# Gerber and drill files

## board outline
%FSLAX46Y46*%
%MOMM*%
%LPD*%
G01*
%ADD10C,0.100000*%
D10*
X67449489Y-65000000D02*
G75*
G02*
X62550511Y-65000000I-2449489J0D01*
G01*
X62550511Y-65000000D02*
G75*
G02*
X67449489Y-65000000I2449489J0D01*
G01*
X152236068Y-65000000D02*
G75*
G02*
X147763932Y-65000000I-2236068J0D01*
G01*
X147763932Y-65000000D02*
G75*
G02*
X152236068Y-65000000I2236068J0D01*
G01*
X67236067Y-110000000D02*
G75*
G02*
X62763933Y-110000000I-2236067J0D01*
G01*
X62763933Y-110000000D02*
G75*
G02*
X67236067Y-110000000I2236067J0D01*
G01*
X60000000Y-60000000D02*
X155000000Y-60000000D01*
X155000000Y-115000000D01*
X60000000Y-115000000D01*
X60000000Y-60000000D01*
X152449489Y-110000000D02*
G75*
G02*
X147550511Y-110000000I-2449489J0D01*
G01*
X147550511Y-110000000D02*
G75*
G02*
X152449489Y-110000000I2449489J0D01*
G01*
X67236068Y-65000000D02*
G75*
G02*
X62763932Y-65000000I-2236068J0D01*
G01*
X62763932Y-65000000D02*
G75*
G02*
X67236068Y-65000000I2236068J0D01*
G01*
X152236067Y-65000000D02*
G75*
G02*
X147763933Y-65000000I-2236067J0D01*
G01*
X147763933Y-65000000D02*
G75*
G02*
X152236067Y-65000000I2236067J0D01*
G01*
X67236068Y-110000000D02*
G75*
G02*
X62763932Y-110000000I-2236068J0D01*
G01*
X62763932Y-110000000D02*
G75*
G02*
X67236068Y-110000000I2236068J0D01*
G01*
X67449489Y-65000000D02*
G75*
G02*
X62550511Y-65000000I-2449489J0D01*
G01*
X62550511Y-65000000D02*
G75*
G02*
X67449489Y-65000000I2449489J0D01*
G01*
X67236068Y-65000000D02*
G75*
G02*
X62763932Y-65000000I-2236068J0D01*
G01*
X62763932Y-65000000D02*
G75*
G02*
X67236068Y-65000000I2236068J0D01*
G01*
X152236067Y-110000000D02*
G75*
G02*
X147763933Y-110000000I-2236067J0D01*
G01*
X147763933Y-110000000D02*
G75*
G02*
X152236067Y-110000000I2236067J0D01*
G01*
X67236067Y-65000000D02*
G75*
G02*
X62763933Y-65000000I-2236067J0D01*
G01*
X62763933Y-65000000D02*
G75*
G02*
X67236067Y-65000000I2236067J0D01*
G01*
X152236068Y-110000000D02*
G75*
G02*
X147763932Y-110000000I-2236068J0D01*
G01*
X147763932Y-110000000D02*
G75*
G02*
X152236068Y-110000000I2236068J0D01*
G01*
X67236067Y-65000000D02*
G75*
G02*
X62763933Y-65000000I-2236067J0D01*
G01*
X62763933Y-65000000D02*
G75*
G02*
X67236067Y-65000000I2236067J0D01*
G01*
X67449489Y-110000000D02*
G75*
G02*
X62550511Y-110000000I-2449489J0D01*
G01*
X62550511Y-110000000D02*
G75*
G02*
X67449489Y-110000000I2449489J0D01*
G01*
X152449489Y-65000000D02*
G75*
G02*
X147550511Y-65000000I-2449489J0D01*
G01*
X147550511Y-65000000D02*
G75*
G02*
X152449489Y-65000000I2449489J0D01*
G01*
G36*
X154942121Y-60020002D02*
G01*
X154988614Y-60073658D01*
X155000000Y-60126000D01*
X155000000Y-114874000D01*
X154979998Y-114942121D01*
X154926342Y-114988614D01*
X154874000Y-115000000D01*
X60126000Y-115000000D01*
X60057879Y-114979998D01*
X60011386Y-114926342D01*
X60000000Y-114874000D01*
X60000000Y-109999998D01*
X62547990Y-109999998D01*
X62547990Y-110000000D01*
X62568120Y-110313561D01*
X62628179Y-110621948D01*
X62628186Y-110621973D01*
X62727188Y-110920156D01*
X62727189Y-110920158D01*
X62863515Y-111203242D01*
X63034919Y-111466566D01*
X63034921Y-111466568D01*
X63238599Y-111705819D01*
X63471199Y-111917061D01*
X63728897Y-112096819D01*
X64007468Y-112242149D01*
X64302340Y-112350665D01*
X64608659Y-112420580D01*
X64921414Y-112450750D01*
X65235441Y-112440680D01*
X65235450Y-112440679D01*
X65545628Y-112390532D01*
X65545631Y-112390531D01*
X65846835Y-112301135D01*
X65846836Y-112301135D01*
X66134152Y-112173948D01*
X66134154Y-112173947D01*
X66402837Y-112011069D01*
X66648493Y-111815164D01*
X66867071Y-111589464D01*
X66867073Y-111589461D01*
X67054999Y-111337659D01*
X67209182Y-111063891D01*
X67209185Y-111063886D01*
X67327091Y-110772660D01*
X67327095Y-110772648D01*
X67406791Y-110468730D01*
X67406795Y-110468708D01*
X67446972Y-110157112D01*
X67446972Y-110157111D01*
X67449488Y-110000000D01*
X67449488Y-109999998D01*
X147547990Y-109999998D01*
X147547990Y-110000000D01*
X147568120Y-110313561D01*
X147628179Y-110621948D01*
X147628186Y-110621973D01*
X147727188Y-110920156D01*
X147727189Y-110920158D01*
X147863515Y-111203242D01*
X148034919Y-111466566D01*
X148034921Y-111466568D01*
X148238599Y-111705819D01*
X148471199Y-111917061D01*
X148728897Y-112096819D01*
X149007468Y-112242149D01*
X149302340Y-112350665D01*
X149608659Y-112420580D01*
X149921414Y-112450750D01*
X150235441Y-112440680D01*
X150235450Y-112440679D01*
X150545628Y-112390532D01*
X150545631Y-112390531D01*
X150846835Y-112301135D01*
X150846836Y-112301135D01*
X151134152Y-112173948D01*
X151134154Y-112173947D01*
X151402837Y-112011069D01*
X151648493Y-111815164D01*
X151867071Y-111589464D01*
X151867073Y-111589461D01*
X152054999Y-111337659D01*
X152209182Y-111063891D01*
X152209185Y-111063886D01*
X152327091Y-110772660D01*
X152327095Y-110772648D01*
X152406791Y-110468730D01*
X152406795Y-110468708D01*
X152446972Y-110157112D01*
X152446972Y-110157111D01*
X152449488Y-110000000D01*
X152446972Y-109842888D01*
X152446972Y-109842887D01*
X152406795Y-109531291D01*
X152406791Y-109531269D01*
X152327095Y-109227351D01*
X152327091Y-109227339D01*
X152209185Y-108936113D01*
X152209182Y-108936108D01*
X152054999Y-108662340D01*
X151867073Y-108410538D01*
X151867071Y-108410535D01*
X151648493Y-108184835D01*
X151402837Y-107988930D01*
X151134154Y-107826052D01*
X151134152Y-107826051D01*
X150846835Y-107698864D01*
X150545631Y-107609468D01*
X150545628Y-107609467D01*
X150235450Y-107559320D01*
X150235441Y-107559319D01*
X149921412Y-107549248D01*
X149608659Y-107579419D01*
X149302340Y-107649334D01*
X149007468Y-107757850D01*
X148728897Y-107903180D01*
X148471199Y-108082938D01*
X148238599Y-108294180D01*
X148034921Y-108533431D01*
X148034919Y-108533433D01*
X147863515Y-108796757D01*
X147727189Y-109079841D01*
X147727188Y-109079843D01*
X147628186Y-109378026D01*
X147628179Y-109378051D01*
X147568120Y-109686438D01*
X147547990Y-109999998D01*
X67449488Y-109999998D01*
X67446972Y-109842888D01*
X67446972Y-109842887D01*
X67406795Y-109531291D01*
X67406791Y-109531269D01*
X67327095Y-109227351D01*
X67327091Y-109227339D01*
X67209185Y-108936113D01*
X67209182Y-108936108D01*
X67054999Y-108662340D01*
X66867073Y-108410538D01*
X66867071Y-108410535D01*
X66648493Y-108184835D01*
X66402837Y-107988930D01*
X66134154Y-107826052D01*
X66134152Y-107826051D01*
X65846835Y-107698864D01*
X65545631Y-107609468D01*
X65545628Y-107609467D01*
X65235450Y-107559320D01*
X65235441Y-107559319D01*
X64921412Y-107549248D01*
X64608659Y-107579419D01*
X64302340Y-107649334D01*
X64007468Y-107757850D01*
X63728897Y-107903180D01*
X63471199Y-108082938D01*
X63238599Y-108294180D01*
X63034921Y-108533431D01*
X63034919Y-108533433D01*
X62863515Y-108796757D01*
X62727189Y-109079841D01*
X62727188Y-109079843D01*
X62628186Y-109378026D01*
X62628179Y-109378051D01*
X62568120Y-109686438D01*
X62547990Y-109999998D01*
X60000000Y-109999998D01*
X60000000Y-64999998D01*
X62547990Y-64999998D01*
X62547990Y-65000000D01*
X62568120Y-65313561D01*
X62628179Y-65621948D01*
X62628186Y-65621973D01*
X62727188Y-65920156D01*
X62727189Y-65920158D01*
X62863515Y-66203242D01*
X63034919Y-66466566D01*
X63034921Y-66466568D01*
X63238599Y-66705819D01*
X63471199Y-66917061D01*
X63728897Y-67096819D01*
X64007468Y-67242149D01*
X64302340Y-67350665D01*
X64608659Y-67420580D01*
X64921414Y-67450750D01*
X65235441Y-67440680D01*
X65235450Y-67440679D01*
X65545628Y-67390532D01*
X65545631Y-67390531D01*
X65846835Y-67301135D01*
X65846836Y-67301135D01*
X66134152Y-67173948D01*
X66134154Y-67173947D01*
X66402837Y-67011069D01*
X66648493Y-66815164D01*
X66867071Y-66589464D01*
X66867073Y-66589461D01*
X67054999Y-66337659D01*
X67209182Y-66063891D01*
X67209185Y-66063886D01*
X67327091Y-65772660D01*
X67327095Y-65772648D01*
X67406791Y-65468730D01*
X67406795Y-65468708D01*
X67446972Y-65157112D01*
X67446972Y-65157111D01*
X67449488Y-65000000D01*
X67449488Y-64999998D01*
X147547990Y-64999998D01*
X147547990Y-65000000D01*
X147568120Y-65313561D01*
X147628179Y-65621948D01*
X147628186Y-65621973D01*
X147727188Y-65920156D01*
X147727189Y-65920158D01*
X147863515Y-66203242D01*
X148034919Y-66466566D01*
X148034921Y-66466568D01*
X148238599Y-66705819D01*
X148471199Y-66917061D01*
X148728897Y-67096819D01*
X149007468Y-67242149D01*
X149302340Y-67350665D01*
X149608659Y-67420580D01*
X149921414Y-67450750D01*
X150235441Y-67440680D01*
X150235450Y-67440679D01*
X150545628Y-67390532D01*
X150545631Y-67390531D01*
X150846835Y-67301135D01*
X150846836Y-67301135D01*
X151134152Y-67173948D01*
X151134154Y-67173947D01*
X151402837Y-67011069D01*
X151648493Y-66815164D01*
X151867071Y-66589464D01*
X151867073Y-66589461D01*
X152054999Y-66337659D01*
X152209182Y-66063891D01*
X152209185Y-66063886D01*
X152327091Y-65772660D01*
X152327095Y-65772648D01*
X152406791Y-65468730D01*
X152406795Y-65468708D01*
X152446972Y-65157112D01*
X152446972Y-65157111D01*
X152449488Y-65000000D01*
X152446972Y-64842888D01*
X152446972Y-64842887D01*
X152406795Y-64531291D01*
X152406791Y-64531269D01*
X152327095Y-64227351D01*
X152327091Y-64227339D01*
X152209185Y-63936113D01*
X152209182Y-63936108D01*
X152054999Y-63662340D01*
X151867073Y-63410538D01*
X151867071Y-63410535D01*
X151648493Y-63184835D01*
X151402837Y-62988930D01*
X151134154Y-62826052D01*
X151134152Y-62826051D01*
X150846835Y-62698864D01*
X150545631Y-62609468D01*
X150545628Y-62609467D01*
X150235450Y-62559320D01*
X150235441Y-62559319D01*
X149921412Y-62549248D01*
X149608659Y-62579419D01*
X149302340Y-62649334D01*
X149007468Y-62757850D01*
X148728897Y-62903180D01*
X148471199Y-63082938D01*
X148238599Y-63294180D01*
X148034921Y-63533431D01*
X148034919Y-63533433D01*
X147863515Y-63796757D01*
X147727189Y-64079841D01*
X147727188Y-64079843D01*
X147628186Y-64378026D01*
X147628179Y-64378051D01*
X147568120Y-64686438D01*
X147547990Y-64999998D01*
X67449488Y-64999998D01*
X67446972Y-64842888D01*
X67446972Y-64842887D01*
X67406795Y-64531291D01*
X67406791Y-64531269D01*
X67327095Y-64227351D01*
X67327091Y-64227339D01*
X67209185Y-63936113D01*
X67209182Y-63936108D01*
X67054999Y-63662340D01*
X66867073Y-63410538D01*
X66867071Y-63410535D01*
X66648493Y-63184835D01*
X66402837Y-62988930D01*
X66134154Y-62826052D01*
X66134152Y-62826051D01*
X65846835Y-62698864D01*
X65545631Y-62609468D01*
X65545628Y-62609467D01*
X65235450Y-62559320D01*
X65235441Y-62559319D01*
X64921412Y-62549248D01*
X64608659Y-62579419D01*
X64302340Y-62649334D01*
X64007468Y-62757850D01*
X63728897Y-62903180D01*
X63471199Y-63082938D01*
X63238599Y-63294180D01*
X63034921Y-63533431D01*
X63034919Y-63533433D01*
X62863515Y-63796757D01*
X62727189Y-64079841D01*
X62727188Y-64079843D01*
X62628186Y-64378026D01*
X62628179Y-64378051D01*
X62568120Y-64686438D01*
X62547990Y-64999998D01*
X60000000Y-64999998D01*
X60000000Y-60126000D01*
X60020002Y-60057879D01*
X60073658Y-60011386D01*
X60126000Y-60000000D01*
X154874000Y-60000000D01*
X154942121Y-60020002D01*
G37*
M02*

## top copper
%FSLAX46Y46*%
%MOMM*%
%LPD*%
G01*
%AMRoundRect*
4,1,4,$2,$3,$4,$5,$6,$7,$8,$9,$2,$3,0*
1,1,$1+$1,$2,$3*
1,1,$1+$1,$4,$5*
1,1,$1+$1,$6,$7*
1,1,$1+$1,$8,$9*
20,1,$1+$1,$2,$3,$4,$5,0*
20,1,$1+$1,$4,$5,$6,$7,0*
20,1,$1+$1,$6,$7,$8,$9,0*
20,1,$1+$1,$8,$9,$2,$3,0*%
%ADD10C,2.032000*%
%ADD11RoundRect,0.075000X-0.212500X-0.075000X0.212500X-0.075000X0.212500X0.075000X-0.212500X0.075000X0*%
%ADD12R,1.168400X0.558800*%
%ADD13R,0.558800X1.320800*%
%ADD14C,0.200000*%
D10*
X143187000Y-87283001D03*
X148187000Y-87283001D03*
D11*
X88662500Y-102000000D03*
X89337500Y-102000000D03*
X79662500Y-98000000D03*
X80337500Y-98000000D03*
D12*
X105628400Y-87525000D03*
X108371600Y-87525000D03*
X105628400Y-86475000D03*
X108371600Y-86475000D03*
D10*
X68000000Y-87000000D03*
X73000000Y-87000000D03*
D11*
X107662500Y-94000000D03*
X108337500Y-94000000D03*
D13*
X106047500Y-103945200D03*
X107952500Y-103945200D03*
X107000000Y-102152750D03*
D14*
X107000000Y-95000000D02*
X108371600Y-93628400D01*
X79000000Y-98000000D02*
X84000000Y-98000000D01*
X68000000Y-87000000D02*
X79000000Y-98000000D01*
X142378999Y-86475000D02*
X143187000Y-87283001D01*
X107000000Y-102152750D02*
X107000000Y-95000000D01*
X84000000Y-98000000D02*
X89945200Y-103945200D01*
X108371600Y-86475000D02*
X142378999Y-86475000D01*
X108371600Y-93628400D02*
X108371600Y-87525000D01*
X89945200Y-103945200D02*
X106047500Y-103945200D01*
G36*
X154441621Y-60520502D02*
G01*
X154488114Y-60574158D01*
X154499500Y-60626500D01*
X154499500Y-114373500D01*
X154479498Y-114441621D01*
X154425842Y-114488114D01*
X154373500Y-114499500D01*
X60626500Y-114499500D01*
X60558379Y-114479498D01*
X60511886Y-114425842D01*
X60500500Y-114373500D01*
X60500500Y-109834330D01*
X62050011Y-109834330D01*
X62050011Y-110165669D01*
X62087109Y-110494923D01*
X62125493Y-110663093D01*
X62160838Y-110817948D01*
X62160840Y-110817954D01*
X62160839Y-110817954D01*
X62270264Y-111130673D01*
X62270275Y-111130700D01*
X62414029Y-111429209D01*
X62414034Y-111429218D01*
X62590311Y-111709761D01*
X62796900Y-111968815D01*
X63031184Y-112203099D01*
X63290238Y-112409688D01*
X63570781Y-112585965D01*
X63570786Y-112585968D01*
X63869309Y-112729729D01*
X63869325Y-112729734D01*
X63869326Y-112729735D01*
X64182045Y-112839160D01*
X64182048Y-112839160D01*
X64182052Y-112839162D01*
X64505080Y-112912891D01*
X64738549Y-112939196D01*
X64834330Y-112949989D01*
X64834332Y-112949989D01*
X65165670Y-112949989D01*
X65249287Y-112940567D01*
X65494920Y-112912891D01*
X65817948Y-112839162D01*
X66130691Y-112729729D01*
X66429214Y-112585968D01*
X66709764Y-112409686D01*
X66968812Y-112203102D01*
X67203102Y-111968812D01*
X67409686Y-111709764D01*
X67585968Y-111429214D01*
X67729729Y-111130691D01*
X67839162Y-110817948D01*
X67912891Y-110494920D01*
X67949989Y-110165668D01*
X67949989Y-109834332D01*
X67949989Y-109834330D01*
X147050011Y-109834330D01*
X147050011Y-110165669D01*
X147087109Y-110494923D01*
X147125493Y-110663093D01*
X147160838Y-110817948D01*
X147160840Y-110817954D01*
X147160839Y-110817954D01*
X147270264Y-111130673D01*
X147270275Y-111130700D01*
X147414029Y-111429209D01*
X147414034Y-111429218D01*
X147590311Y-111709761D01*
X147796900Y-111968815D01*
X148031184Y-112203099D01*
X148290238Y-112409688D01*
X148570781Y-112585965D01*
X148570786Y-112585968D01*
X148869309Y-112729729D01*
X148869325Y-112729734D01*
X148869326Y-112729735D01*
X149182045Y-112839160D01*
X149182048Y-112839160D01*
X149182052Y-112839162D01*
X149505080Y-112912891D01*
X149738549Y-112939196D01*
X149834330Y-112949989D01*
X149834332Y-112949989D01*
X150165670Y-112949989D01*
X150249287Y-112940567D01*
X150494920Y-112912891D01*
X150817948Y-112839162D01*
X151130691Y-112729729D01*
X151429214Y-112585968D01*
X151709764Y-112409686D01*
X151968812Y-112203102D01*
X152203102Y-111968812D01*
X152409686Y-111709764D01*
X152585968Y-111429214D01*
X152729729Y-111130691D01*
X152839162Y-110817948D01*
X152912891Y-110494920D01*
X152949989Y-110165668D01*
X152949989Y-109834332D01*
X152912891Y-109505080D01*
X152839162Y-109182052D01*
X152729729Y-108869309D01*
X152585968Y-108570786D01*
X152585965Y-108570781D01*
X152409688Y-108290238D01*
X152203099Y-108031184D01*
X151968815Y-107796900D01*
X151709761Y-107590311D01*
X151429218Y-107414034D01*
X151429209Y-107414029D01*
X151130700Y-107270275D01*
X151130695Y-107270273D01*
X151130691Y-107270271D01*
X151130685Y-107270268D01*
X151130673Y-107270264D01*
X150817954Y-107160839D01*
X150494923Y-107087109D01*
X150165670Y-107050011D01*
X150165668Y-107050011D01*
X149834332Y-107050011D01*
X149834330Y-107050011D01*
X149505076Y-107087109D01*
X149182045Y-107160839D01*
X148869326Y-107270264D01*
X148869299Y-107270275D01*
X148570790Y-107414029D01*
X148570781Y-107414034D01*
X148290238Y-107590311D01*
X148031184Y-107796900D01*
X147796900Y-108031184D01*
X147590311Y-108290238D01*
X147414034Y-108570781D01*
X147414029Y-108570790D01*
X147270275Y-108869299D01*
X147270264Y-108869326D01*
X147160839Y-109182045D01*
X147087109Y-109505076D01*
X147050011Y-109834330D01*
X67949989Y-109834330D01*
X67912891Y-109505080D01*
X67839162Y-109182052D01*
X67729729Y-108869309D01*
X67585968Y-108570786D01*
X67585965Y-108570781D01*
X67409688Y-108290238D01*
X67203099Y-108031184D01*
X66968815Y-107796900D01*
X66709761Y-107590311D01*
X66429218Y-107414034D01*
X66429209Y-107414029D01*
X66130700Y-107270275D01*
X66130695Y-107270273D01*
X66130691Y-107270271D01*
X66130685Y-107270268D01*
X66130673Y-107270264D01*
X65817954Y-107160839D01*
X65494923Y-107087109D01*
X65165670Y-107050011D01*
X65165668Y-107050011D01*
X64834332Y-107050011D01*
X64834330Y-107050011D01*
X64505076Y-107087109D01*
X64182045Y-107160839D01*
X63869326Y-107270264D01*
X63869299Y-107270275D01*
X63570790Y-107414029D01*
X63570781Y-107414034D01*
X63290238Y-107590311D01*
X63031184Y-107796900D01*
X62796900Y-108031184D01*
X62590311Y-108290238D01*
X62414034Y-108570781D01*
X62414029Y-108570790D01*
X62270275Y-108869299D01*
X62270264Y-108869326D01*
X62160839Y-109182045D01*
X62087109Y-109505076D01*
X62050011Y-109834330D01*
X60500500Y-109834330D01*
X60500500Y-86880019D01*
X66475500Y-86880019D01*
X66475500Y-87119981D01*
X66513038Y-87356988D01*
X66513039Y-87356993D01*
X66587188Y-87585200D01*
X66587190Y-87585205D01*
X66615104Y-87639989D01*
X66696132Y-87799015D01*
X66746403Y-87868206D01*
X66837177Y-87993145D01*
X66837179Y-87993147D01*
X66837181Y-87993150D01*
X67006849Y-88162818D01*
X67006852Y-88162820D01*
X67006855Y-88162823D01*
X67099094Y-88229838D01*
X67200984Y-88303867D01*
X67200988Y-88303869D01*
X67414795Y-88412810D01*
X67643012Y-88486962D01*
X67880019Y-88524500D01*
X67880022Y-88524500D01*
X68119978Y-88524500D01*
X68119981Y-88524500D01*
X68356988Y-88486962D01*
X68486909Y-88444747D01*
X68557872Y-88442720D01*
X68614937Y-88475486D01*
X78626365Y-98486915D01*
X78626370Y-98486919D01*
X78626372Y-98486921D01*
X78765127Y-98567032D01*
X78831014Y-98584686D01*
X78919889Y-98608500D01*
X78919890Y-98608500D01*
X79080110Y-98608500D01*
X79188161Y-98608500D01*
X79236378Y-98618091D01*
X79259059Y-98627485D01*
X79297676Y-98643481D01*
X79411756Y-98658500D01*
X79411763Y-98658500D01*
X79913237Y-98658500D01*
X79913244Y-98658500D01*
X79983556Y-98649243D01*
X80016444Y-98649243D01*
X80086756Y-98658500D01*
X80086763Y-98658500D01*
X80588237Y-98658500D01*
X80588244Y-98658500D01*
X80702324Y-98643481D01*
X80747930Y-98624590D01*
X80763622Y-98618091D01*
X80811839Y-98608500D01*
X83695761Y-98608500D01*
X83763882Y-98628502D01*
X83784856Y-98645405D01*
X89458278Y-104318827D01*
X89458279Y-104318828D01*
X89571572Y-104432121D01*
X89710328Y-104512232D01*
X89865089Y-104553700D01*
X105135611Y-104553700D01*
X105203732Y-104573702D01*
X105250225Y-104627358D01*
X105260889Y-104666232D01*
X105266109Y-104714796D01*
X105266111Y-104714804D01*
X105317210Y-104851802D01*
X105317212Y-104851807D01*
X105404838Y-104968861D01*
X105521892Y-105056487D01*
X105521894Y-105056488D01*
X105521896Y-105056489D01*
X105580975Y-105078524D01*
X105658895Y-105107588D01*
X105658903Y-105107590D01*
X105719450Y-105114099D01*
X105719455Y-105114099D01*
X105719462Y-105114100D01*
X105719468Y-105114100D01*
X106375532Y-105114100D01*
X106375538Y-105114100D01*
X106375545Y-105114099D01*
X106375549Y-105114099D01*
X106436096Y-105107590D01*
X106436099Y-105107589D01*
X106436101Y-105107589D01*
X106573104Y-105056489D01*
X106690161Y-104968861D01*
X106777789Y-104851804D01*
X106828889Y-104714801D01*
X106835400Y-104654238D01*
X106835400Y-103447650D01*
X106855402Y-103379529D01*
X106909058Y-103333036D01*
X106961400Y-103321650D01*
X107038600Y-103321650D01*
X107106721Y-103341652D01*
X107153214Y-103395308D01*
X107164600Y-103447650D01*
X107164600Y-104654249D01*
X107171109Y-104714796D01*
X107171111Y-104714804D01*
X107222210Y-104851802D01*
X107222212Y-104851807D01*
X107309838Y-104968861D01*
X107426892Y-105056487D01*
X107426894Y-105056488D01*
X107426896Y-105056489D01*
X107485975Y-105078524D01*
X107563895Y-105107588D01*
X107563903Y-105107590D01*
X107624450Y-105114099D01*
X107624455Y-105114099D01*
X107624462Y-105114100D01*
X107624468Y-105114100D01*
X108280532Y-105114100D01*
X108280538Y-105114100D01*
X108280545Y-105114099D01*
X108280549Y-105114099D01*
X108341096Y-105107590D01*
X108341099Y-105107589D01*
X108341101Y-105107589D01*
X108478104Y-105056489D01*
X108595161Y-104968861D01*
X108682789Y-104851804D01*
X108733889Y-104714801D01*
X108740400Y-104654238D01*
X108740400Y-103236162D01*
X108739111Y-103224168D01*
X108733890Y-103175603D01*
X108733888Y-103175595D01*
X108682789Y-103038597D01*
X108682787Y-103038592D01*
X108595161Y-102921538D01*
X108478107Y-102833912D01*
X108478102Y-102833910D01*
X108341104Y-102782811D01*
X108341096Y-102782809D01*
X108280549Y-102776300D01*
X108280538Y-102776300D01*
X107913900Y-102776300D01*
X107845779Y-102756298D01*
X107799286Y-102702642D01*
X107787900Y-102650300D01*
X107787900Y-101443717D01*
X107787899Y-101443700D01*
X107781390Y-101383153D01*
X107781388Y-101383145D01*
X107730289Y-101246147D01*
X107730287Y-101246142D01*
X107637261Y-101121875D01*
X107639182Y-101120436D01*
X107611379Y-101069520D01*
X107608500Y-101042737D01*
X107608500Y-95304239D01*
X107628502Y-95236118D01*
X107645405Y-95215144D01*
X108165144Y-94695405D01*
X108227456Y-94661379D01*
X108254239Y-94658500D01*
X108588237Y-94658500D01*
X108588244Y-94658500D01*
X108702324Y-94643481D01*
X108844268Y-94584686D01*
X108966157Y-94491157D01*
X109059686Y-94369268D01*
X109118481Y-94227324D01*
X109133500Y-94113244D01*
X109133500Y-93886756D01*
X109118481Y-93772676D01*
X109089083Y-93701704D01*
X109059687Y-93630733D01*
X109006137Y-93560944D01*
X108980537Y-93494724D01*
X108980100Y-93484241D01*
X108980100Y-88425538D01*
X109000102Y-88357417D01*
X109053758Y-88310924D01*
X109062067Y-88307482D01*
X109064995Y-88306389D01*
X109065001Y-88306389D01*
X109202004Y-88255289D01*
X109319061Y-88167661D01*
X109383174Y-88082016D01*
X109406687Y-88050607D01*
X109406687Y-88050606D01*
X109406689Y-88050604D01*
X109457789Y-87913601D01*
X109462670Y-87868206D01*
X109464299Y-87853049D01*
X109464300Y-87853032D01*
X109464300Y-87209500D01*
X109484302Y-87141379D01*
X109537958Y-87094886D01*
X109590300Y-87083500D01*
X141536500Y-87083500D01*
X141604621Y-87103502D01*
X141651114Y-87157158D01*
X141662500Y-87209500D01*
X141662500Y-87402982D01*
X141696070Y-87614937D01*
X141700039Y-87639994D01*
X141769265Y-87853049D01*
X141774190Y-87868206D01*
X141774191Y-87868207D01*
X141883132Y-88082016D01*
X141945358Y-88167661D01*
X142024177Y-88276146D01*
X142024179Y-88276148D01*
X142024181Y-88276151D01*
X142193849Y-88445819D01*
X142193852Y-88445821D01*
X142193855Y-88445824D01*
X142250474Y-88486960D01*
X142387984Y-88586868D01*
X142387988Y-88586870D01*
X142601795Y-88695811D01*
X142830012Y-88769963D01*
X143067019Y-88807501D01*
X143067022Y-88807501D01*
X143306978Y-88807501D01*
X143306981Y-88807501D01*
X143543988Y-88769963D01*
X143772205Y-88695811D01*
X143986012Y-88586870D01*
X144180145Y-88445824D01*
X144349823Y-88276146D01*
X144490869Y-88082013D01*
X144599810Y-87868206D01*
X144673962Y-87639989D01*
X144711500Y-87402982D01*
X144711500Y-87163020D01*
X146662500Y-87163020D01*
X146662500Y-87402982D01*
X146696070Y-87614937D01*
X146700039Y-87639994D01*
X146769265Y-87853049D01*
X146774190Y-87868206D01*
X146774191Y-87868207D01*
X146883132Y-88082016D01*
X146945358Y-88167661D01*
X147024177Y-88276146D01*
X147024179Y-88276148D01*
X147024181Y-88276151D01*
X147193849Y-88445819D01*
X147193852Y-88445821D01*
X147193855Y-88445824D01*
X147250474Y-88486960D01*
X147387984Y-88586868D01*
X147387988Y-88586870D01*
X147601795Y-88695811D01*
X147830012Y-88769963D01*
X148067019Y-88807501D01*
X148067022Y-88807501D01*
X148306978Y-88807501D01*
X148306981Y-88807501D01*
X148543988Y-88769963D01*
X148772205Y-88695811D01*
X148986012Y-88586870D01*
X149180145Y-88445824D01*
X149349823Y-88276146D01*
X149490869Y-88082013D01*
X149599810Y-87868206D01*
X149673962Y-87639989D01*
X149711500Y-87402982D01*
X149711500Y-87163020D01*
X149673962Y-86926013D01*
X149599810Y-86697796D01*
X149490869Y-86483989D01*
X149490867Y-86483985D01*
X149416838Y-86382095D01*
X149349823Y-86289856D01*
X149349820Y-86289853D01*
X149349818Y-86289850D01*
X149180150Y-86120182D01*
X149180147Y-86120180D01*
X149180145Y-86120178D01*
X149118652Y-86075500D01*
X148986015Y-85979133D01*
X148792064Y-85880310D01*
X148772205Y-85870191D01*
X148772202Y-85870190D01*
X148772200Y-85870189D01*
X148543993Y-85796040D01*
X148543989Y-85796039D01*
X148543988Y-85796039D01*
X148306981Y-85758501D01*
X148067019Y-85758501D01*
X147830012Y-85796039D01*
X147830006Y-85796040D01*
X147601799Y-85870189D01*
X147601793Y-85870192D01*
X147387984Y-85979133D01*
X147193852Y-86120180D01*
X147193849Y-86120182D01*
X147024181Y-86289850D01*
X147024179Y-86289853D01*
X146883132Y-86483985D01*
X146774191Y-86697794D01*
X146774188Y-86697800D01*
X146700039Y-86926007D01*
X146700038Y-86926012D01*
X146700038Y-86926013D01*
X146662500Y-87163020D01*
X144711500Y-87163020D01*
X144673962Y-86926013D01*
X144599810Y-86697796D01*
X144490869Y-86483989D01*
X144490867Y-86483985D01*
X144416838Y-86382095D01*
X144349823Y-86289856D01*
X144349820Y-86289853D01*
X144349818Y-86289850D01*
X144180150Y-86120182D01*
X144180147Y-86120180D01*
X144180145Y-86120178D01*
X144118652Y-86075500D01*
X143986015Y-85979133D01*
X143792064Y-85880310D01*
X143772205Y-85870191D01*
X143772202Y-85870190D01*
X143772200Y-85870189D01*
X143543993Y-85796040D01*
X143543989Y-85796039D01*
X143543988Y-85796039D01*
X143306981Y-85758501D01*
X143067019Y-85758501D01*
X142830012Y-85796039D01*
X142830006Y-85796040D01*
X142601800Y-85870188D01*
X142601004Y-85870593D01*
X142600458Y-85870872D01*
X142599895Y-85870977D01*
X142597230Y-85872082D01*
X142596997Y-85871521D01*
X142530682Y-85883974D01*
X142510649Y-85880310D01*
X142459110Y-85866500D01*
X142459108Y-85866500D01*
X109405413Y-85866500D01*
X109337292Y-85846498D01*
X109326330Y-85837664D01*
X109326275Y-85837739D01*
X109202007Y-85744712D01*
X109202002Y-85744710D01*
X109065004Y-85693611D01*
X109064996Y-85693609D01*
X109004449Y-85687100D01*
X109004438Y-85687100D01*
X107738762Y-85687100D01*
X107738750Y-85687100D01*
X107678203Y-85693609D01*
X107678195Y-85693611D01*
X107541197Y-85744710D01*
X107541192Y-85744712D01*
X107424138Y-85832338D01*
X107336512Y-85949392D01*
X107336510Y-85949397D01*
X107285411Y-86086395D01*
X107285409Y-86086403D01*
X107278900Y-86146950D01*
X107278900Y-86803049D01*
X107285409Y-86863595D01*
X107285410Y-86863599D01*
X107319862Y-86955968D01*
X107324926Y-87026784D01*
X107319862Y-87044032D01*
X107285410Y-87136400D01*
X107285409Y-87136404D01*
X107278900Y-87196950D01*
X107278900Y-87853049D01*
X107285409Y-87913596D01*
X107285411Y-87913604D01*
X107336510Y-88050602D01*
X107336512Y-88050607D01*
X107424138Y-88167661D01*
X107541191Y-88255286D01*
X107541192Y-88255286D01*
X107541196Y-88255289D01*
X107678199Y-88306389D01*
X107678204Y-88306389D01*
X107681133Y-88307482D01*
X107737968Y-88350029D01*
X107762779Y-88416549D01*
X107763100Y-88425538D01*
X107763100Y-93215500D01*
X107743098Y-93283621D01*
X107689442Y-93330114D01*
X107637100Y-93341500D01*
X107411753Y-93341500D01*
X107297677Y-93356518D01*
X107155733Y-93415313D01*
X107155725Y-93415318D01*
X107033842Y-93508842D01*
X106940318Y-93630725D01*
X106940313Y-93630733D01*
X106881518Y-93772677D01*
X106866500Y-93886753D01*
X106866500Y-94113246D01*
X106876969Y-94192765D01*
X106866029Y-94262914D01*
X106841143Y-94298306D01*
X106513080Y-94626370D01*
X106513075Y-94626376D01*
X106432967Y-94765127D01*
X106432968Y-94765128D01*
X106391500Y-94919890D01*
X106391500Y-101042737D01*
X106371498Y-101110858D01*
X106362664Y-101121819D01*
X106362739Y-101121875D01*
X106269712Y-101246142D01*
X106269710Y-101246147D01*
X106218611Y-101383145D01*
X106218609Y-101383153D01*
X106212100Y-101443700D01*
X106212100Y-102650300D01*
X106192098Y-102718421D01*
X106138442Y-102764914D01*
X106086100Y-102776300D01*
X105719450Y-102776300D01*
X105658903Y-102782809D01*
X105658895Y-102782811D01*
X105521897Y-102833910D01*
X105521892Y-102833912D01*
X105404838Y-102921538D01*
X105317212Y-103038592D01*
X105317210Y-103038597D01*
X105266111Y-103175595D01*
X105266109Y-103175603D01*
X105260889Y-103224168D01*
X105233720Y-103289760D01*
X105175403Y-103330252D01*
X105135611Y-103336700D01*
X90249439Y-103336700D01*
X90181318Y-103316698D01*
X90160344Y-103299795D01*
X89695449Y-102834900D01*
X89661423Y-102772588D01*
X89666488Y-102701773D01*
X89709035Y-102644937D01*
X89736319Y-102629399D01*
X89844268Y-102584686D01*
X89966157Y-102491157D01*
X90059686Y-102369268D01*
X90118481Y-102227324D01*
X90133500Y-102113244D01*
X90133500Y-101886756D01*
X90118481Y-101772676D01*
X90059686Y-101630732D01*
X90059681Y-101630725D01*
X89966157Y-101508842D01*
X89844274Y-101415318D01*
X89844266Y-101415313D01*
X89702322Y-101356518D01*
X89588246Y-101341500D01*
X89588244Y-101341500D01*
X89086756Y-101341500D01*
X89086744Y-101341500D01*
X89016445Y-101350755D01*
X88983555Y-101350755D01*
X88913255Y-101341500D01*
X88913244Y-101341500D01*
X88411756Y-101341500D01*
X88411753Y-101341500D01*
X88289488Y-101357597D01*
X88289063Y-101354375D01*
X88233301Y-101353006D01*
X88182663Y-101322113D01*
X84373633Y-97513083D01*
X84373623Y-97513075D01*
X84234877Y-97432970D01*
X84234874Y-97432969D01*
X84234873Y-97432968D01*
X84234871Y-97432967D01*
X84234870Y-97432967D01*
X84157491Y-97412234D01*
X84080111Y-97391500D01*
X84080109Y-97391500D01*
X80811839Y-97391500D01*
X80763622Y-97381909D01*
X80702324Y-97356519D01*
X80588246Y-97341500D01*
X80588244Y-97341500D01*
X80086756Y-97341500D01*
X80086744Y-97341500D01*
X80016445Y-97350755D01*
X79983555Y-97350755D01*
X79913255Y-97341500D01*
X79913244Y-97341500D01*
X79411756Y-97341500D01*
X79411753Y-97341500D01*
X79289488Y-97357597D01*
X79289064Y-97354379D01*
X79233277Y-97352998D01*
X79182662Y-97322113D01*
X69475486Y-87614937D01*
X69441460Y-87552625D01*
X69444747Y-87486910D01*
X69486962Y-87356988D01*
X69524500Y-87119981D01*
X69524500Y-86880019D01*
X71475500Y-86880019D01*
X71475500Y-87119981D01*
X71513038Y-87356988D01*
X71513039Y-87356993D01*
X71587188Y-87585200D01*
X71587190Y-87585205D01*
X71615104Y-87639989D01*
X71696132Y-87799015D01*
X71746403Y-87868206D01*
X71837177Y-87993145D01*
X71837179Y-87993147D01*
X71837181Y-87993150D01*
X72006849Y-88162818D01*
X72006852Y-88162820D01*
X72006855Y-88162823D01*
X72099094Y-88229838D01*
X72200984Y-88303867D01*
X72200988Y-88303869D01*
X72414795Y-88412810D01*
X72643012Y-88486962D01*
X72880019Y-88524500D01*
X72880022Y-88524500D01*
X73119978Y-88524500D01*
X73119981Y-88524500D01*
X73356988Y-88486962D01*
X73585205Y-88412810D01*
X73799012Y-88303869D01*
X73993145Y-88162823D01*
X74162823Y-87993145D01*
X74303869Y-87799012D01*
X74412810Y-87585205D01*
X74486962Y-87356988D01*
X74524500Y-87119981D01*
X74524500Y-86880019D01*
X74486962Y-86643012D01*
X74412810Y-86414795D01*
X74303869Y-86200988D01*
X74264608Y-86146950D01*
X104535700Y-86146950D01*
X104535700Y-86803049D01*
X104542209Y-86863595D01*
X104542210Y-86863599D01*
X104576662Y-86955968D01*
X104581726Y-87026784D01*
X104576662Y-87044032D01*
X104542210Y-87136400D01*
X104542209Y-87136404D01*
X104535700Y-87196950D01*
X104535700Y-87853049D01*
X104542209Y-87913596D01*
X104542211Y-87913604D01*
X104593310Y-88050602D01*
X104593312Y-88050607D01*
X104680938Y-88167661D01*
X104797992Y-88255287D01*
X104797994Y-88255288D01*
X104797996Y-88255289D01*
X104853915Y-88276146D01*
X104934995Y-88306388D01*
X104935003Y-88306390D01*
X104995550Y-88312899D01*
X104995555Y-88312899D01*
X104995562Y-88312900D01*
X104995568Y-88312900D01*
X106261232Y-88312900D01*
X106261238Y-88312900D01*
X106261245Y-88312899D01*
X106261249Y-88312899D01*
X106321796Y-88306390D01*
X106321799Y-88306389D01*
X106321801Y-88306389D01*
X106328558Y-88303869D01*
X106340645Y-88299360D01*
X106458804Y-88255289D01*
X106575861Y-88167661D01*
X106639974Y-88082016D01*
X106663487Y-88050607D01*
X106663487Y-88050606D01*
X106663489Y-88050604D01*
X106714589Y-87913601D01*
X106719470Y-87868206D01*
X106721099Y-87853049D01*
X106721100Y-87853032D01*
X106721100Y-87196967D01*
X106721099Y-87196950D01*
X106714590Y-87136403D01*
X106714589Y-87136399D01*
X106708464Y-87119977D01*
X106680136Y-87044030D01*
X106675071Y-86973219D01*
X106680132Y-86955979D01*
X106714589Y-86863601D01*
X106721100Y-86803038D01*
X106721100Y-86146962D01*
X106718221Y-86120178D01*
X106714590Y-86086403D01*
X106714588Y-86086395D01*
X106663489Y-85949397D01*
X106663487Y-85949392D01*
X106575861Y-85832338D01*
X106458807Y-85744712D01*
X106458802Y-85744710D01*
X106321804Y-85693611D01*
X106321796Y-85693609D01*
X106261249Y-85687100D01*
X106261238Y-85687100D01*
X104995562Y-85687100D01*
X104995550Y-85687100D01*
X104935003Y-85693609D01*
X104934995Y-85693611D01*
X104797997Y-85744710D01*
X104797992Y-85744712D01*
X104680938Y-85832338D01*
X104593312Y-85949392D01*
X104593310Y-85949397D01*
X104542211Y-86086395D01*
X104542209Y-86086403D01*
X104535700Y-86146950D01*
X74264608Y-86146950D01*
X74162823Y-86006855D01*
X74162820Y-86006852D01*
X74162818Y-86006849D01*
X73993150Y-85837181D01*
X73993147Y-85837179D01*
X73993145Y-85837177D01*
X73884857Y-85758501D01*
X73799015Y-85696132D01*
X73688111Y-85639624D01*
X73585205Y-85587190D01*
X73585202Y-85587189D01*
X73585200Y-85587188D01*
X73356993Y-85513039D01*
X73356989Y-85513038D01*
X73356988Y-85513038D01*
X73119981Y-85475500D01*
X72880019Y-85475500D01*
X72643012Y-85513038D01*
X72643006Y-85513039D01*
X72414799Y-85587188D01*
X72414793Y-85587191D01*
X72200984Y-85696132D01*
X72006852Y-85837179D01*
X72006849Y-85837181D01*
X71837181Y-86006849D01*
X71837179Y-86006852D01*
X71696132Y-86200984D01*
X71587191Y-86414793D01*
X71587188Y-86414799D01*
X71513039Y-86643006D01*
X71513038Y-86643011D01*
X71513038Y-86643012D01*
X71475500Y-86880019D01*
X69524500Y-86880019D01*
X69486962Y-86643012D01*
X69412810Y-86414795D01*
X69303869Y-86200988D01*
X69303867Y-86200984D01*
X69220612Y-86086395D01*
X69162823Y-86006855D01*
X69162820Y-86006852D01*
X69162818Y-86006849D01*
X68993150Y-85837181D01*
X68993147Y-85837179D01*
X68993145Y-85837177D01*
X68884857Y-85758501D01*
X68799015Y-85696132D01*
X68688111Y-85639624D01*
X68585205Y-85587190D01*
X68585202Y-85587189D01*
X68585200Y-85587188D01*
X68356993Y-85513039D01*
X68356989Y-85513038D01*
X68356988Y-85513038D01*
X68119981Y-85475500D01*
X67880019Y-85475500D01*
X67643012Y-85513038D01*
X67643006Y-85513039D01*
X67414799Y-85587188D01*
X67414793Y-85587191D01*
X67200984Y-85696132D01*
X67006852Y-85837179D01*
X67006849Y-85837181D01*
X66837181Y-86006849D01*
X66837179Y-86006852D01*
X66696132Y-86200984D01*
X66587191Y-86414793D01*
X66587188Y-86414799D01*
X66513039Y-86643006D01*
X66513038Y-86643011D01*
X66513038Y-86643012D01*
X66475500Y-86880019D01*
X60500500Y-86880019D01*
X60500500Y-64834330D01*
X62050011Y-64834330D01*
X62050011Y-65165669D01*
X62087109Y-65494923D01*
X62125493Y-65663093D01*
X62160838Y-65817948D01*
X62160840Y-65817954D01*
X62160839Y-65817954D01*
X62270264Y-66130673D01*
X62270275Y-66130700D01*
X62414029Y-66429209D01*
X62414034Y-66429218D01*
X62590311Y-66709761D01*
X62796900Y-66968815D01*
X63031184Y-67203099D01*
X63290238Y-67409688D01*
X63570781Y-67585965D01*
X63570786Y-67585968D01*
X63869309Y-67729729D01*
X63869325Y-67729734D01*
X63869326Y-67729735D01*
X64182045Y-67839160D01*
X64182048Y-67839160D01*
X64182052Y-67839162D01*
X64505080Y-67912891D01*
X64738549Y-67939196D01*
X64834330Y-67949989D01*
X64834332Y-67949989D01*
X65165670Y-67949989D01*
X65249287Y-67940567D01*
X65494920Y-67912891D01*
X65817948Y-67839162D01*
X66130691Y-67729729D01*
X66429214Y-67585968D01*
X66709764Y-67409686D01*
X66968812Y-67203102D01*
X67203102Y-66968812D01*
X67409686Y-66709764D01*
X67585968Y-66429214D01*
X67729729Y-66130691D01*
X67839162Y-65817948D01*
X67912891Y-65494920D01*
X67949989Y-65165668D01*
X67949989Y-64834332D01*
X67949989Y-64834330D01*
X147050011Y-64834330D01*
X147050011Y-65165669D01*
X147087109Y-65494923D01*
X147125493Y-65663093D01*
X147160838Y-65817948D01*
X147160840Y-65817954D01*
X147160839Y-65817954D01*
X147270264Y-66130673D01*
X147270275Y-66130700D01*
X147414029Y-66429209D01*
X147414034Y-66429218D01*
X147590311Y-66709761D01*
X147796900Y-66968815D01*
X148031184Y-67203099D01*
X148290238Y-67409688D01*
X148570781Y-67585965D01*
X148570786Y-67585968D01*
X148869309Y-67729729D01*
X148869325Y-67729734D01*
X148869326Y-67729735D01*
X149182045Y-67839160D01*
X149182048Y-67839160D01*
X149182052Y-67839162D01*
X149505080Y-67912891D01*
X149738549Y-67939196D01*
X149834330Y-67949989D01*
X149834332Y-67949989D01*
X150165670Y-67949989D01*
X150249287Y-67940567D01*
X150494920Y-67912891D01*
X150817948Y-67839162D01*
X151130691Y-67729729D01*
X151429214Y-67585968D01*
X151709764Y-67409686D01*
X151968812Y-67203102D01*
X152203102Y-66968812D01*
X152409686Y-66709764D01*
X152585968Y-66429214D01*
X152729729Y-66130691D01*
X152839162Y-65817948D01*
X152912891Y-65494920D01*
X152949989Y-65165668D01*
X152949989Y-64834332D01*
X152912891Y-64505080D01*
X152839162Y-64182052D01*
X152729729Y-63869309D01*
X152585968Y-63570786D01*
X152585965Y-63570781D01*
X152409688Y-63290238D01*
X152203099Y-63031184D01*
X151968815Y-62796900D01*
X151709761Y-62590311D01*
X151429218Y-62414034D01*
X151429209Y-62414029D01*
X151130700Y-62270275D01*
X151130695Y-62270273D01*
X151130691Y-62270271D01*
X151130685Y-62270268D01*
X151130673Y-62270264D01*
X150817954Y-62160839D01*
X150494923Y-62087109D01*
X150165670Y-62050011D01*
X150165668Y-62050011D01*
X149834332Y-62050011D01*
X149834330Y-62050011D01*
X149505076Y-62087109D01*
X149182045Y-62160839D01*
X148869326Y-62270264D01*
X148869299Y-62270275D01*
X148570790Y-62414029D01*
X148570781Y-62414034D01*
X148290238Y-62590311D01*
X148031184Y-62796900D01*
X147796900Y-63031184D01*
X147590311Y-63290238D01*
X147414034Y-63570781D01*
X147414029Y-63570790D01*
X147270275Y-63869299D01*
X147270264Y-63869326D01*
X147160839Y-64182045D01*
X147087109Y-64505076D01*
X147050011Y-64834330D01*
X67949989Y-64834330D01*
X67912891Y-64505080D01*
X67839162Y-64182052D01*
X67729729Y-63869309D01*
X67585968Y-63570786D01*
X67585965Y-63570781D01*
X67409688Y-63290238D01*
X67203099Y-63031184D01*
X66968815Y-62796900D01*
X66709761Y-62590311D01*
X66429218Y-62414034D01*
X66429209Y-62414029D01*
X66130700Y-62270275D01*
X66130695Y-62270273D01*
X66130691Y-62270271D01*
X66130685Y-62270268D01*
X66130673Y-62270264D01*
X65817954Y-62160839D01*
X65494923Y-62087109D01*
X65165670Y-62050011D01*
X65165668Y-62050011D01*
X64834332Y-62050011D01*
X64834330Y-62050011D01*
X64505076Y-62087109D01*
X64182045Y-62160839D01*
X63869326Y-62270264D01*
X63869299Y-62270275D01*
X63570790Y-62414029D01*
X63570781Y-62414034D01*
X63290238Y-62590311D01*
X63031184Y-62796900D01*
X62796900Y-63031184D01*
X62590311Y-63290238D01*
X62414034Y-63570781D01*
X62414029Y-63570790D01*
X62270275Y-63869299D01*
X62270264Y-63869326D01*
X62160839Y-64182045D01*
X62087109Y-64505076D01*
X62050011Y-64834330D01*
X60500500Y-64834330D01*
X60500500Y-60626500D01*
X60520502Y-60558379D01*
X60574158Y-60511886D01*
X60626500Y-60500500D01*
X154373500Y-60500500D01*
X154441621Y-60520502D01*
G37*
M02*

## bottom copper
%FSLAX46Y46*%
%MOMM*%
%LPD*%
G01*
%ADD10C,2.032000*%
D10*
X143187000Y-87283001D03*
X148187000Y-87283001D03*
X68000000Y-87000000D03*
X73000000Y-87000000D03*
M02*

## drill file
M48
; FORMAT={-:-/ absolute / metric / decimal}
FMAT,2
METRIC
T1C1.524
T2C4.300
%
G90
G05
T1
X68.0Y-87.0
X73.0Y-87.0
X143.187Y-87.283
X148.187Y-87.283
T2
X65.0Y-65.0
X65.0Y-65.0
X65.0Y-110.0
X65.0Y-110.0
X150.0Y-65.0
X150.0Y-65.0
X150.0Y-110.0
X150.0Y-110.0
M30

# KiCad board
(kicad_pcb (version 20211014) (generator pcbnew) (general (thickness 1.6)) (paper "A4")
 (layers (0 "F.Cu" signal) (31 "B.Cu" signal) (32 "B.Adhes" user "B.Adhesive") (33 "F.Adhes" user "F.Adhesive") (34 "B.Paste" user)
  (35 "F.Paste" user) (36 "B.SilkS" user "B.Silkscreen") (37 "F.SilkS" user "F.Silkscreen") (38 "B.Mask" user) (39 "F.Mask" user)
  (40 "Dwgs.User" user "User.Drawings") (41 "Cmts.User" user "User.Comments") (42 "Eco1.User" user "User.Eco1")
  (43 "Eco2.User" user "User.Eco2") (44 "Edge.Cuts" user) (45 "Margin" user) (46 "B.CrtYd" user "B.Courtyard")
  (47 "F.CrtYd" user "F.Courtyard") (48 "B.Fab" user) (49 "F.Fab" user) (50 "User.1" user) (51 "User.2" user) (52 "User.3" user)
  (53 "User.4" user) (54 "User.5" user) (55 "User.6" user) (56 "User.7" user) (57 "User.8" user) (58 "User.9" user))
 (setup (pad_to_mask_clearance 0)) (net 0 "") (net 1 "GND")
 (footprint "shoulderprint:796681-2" (layer "F.Cu") (at 143.187 87.283001)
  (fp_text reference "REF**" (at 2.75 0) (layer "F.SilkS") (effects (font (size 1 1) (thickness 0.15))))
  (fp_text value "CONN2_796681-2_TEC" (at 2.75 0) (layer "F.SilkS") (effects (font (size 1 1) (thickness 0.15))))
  (pad "1" thru_hole circle locked (at 0 0) (size 2.032 2.032) (drill 1.524) (layers *.Cu *.Mask))
  (pad "2" thru_hole circle locked (at 5 0) (size 2.032 2.032) (drill 1.524) (layers *.Cu *.Mask)))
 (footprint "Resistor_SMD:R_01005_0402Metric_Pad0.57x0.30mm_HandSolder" (layer "F.Cu") (at 89 102)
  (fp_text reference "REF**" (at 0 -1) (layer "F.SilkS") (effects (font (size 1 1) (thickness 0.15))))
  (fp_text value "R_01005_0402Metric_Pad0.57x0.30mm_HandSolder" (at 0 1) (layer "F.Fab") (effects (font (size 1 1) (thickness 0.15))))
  (pad "" smd roundrect (at -0.3625 0) (size 0.41 0.27) (layers "F.Paste") (roundrect_rratio 0.25))
  (pad "" smd roundrect (at 0.3625 0) (size 0.41 0.27) (layers "F.Paste") (roundrect_rratio 0.25))
  (pad "1" smd roundrect (at -0.3375 0) (size 0.575 0.3) (layers "F.Cu" "F.Mask") (roundrect_rratio 0.25))
  (pad "2" smd roundrect (at 0.3375 0) (size 0.575 0.3) (layers "F.Cu" "F.Mask") (roundrect_rratio 0.25)))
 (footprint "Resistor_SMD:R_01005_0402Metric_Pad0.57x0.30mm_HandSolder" (layer "F.Cu") (at 80 98)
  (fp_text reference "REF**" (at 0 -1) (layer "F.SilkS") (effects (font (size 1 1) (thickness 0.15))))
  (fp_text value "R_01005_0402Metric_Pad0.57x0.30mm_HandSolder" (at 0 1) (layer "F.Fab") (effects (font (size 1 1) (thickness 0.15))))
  (pad "" smd roundrect (at 0.3625 0) (size 0.41 0.27) (layers "F.Paste") (roundrect_rratio 0.25))
  (pad "" smd roundrect (at -0.3625 0) (size 0.41 0.27) (layers "F.Paste") (roundrect_rratio 0.25))
  (pad "1" smd roundrect (at -0.3375 0) (size 0.575 0.3) (layers "F.Cu" "F.Mask") (roundrect_rratio 0.25))
  (pad "2" smd roundrect (at 0.3375 0) (size 0.575 0.3) (layers "F.Cu" "F.Mask") (roundrect_rratio 0.25)))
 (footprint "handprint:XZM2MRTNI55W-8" (layer "F.Cu") (at 107 87)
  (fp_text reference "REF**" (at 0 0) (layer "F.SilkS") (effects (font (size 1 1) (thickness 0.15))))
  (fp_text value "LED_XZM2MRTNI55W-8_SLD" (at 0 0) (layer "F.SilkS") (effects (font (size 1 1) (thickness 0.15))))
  (pad "1" smd rect locked (at -1.3716 0.525) (size 1.1684 0.5588) (layers "F.Cu" "F.Paste" "F.Mask"))
  (pad "2" smd rect locked (at 1.3716 0.525) (size 1.1684 0.5588) (layers "F.Cu" "F.Paste" "F.Mask"))
  (pad "3" smd rect locked (at -1.3716 -0.525) (size 1.1684 0.5588) (layers "F.Cu" "F.Paste" "F.Mask"))
  (pad "4" smd rect locked (at 1.3716 -0.525) (size 1.1684 0.5588) (layers "F.Cu" "F.Paste" "F.Mask")))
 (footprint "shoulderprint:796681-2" (layer "F.Cu") (at 68 87)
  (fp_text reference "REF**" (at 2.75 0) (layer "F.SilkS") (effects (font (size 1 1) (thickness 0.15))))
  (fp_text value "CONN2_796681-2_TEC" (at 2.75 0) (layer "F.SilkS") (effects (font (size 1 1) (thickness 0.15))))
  (pad "1" thru_hole circle locked (at 0 0) (size 2.032 2.032) (drill 1.524) (layers *.Cu *.Mask))
  (pad "2" thru_hole circle locked (at 5 0) (size 2.032 2.032) (drill 1.524) (layers *.Cu *.Mask)))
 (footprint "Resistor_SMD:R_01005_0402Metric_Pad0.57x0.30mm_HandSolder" (layer "F.Cu") (at 108 94)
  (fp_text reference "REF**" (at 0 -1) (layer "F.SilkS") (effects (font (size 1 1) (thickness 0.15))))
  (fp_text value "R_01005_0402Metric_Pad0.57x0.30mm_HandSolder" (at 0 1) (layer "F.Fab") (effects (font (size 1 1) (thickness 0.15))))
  (pad "" smd roundrect (at -0.3625 0) (size 0.41 0.27) (layers "F.Paste") (roundrect_rratio 0.25))
  (pad "" smd roundrect (at 0.3625 0) (size 0.41 0.27) (layers "F.Paste") (roundrect_rratio 0.25))
  (pad "1" smd roundrect (at -0.3375 0) (size 0.575 0.3) (layers "F.Cu" "F.Mask") (roundrect_rratio 0.25))
  (pad "2" smd roundrect (at 0.3375 0) (size 0.575 0.3) (layers "F.Cu" "F.Mask") (roundrect_rratio 0.25)))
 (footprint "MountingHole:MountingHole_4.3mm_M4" (layer "F.Cu") (at 65 110)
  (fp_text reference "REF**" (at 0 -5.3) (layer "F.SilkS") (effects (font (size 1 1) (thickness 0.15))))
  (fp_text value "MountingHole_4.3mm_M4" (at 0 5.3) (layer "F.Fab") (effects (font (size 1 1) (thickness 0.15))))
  (pad "" np_thru_hole circle (at 0 0) (size 4.3 4.3) (drill 4.3) (layers *.Cu *.Mask))
  (pad "" np_thru_hole circle (at 0 0) (size 4.3 4.3) (drill 4.3) (layers *.Cu *.Mask)))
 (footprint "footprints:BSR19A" (layer "F.Cu") (at 107 103)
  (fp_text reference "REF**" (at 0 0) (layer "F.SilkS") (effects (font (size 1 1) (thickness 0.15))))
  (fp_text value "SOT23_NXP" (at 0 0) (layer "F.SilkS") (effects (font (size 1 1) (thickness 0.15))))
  (pad "1" smd rect (at -0.9525 0.9452) (size 0.5588 1.3208) (layers "F.Cu" "F.Paste" "F.Mask"))
  (pad "2" smd rect (at 0.9525 0.9452) (size 0.5588 1.3208) (layers "F.Cu" "F.Paste" "F.Mask"))
  (pad "3" smd rect (at 0 -0.84725) (size 0.5588 1.3208) (layers "F.Cu" "F.Paste" "F.Mask")))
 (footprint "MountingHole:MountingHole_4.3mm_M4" (layer "F.Cu") (at 65 65)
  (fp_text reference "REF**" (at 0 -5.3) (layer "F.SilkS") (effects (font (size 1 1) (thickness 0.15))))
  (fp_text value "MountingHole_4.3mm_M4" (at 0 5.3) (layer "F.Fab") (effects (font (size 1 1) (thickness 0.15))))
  (pad "" np_thru_hole circle (at 0 0) (size 4.3 4.3) (drill 4.3) (layers *.Cu *.Mask))
  (pad "" np_thru_hole circle (at 0 0) (size 4.3 4.3) (drill 4.3) (layers *.Cu *.Mask)))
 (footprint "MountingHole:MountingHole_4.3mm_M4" (layer "F.Cu") (at 150 110)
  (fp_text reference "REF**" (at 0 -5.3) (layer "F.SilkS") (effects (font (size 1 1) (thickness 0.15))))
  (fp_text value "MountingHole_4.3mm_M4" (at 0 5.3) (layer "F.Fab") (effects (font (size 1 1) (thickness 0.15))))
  (pad "" np_thru_hole circle (at 0 0) (size 4.3 4.3) (drill 4.3) (layers *.Cu *.Mask))
  (pad "" np_thru_hole circle (at 0 0) (size 4.3 4.3) (drill 4.3) (layers *.Cu *.Mask)))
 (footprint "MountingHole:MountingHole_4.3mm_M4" (layer "F.Cu") (at 150 65)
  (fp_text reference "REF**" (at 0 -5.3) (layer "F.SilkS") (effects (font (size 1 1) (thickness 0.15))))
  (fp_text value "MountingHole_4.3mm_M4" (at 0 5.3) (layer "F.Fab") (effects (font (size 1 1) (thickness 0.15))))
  (pad "" np_thru_hole circle (at 0 0) (size 4.3 4.3) (drill 4.3) (layers *.Cu *.Mask))
  (pad "" np_thru_hole circle (at 0 0) (size 4.3 4.3) (drill 4.3) (layers *.Cu *.Mask)))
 (gr_circle (center 65 65) (end 67.236067 66) (layer "Edge.Cuts") (width 0.1) (fill none))
 (gr_circle (center 150 65) (end 151 67) (layer "Edge.Cuts") (width 0.1) (fill none))
 (gr_circle (center 65 110) (end 65 112.236067) (layer "Edge.Cuts") (width 0.1) (fill none))
 (gr_rect (start 60 60) (end 155 115) (layer "Edge.Cuts") (width 0.1) (fill none))
 (gr_circle (center 150 110) (end 152.236067 111) (layer "Edge.Cuts") (width 0.1) (fill none))
 (gr_circle (center 65 65) (end 66 67) (layer "Edge.Cuts") (width 0.1) (fill none))
 (gr_circle (center 150 65) (end 150 67.236067) (layer "Edge.Cuts") (width 0.1) (fill none))
 (gr_circle (center 65 110) (end 66 112) (layer "Edge.Cuts") (width 0.1) (fill none))
 (gr_circle (center 65 65) (end 67.236067 66) (layer "Edge.Cuts") (width 0.1) (fill none))
 (gr_circle (center 65 65) (end 66 67) (layer "Edge.Cuts") (width 0.1) (fill none))
 (gr_circle (center 150 110) (end 150 112.236067) (layer "Edge.Cuts") (width 0.1) (fill none))
 (gr_circle (center 65 65) (end 65 67.236067) (layer "Edge.Cuts") (width 0.1) (fill none))
 (gr_circle (center 150 110) (end 151 112) (layer "Edge.Cuts") (width 0.1) (fill none))
 (gr_circle (center 65 65) (end 65 67.236067) (layer "Edge.Cuts") (width 0.1) (fill none))
 (gr_circle (center 65 110) (end 67.236067 111) (layer "Edge.Cuts") (width 0.1) (fill none))
 (gr_circle (center 150 65) (end 152.236067 66) (layer "Edge.Cuts") (width 0.1) (fill none))
 (segment (start 107 95) (end 108.3716 93.6284) (width 0.2) (layer "F.Cu") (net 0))
 (segment (start 79 98) (end 84 98) (width 0.2) (layer "F.Cu") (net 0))
 (segment (start 68 87) (end 79 98) (width 0.2) (layer "F.Cu") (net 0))
 (segment (start 142.378999 86.475) (end 143.187 87.283001) (width 0.2) (layer "F.Cu") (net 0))
 (segment (start 107 102.15275) (end 107 95) (width 0.2) (layer "F.Cu") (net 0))
 (segment (start 84 98) (end 89.9452 103.9452) (width 0.2) (layer "F.Cu") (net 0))
 (segment (start 108.3716 86.475) (end 142.378999 86.475) (width 0.2) (layer "F.Cu") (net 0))
 (segment (start 108.3716 93.6284) (end 108.3716 87.525) (width 0.2) (layer "F.Cu") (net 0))
 (segment (start 89.9452 103.9452) (end 106.0475 103.9452) (width 0.2) (layer "F.Cu") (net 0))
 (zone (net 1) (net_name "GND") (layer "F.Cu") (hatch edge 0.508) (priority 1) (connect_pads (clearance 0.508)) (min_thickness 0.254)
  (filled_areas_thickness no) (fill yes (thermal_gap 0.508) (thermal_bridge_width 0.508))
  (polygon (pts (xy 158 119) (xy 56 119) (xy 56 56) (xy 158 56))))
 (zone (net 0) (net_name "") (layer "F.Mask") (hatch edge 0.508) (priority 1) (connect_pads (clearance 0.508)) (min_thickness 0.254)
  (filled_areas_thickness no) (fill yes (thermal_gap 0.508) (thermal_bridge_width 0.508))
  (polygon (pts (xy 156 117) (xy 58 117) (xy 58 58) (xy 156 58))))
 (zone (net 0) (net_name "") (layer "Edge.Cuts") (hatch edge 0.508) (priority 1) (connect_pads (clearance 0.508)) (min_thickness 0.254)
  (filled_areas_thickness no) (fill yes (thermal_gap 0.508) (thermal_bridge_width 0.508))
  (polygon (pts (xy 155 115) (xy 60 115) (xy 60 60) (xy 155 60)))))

